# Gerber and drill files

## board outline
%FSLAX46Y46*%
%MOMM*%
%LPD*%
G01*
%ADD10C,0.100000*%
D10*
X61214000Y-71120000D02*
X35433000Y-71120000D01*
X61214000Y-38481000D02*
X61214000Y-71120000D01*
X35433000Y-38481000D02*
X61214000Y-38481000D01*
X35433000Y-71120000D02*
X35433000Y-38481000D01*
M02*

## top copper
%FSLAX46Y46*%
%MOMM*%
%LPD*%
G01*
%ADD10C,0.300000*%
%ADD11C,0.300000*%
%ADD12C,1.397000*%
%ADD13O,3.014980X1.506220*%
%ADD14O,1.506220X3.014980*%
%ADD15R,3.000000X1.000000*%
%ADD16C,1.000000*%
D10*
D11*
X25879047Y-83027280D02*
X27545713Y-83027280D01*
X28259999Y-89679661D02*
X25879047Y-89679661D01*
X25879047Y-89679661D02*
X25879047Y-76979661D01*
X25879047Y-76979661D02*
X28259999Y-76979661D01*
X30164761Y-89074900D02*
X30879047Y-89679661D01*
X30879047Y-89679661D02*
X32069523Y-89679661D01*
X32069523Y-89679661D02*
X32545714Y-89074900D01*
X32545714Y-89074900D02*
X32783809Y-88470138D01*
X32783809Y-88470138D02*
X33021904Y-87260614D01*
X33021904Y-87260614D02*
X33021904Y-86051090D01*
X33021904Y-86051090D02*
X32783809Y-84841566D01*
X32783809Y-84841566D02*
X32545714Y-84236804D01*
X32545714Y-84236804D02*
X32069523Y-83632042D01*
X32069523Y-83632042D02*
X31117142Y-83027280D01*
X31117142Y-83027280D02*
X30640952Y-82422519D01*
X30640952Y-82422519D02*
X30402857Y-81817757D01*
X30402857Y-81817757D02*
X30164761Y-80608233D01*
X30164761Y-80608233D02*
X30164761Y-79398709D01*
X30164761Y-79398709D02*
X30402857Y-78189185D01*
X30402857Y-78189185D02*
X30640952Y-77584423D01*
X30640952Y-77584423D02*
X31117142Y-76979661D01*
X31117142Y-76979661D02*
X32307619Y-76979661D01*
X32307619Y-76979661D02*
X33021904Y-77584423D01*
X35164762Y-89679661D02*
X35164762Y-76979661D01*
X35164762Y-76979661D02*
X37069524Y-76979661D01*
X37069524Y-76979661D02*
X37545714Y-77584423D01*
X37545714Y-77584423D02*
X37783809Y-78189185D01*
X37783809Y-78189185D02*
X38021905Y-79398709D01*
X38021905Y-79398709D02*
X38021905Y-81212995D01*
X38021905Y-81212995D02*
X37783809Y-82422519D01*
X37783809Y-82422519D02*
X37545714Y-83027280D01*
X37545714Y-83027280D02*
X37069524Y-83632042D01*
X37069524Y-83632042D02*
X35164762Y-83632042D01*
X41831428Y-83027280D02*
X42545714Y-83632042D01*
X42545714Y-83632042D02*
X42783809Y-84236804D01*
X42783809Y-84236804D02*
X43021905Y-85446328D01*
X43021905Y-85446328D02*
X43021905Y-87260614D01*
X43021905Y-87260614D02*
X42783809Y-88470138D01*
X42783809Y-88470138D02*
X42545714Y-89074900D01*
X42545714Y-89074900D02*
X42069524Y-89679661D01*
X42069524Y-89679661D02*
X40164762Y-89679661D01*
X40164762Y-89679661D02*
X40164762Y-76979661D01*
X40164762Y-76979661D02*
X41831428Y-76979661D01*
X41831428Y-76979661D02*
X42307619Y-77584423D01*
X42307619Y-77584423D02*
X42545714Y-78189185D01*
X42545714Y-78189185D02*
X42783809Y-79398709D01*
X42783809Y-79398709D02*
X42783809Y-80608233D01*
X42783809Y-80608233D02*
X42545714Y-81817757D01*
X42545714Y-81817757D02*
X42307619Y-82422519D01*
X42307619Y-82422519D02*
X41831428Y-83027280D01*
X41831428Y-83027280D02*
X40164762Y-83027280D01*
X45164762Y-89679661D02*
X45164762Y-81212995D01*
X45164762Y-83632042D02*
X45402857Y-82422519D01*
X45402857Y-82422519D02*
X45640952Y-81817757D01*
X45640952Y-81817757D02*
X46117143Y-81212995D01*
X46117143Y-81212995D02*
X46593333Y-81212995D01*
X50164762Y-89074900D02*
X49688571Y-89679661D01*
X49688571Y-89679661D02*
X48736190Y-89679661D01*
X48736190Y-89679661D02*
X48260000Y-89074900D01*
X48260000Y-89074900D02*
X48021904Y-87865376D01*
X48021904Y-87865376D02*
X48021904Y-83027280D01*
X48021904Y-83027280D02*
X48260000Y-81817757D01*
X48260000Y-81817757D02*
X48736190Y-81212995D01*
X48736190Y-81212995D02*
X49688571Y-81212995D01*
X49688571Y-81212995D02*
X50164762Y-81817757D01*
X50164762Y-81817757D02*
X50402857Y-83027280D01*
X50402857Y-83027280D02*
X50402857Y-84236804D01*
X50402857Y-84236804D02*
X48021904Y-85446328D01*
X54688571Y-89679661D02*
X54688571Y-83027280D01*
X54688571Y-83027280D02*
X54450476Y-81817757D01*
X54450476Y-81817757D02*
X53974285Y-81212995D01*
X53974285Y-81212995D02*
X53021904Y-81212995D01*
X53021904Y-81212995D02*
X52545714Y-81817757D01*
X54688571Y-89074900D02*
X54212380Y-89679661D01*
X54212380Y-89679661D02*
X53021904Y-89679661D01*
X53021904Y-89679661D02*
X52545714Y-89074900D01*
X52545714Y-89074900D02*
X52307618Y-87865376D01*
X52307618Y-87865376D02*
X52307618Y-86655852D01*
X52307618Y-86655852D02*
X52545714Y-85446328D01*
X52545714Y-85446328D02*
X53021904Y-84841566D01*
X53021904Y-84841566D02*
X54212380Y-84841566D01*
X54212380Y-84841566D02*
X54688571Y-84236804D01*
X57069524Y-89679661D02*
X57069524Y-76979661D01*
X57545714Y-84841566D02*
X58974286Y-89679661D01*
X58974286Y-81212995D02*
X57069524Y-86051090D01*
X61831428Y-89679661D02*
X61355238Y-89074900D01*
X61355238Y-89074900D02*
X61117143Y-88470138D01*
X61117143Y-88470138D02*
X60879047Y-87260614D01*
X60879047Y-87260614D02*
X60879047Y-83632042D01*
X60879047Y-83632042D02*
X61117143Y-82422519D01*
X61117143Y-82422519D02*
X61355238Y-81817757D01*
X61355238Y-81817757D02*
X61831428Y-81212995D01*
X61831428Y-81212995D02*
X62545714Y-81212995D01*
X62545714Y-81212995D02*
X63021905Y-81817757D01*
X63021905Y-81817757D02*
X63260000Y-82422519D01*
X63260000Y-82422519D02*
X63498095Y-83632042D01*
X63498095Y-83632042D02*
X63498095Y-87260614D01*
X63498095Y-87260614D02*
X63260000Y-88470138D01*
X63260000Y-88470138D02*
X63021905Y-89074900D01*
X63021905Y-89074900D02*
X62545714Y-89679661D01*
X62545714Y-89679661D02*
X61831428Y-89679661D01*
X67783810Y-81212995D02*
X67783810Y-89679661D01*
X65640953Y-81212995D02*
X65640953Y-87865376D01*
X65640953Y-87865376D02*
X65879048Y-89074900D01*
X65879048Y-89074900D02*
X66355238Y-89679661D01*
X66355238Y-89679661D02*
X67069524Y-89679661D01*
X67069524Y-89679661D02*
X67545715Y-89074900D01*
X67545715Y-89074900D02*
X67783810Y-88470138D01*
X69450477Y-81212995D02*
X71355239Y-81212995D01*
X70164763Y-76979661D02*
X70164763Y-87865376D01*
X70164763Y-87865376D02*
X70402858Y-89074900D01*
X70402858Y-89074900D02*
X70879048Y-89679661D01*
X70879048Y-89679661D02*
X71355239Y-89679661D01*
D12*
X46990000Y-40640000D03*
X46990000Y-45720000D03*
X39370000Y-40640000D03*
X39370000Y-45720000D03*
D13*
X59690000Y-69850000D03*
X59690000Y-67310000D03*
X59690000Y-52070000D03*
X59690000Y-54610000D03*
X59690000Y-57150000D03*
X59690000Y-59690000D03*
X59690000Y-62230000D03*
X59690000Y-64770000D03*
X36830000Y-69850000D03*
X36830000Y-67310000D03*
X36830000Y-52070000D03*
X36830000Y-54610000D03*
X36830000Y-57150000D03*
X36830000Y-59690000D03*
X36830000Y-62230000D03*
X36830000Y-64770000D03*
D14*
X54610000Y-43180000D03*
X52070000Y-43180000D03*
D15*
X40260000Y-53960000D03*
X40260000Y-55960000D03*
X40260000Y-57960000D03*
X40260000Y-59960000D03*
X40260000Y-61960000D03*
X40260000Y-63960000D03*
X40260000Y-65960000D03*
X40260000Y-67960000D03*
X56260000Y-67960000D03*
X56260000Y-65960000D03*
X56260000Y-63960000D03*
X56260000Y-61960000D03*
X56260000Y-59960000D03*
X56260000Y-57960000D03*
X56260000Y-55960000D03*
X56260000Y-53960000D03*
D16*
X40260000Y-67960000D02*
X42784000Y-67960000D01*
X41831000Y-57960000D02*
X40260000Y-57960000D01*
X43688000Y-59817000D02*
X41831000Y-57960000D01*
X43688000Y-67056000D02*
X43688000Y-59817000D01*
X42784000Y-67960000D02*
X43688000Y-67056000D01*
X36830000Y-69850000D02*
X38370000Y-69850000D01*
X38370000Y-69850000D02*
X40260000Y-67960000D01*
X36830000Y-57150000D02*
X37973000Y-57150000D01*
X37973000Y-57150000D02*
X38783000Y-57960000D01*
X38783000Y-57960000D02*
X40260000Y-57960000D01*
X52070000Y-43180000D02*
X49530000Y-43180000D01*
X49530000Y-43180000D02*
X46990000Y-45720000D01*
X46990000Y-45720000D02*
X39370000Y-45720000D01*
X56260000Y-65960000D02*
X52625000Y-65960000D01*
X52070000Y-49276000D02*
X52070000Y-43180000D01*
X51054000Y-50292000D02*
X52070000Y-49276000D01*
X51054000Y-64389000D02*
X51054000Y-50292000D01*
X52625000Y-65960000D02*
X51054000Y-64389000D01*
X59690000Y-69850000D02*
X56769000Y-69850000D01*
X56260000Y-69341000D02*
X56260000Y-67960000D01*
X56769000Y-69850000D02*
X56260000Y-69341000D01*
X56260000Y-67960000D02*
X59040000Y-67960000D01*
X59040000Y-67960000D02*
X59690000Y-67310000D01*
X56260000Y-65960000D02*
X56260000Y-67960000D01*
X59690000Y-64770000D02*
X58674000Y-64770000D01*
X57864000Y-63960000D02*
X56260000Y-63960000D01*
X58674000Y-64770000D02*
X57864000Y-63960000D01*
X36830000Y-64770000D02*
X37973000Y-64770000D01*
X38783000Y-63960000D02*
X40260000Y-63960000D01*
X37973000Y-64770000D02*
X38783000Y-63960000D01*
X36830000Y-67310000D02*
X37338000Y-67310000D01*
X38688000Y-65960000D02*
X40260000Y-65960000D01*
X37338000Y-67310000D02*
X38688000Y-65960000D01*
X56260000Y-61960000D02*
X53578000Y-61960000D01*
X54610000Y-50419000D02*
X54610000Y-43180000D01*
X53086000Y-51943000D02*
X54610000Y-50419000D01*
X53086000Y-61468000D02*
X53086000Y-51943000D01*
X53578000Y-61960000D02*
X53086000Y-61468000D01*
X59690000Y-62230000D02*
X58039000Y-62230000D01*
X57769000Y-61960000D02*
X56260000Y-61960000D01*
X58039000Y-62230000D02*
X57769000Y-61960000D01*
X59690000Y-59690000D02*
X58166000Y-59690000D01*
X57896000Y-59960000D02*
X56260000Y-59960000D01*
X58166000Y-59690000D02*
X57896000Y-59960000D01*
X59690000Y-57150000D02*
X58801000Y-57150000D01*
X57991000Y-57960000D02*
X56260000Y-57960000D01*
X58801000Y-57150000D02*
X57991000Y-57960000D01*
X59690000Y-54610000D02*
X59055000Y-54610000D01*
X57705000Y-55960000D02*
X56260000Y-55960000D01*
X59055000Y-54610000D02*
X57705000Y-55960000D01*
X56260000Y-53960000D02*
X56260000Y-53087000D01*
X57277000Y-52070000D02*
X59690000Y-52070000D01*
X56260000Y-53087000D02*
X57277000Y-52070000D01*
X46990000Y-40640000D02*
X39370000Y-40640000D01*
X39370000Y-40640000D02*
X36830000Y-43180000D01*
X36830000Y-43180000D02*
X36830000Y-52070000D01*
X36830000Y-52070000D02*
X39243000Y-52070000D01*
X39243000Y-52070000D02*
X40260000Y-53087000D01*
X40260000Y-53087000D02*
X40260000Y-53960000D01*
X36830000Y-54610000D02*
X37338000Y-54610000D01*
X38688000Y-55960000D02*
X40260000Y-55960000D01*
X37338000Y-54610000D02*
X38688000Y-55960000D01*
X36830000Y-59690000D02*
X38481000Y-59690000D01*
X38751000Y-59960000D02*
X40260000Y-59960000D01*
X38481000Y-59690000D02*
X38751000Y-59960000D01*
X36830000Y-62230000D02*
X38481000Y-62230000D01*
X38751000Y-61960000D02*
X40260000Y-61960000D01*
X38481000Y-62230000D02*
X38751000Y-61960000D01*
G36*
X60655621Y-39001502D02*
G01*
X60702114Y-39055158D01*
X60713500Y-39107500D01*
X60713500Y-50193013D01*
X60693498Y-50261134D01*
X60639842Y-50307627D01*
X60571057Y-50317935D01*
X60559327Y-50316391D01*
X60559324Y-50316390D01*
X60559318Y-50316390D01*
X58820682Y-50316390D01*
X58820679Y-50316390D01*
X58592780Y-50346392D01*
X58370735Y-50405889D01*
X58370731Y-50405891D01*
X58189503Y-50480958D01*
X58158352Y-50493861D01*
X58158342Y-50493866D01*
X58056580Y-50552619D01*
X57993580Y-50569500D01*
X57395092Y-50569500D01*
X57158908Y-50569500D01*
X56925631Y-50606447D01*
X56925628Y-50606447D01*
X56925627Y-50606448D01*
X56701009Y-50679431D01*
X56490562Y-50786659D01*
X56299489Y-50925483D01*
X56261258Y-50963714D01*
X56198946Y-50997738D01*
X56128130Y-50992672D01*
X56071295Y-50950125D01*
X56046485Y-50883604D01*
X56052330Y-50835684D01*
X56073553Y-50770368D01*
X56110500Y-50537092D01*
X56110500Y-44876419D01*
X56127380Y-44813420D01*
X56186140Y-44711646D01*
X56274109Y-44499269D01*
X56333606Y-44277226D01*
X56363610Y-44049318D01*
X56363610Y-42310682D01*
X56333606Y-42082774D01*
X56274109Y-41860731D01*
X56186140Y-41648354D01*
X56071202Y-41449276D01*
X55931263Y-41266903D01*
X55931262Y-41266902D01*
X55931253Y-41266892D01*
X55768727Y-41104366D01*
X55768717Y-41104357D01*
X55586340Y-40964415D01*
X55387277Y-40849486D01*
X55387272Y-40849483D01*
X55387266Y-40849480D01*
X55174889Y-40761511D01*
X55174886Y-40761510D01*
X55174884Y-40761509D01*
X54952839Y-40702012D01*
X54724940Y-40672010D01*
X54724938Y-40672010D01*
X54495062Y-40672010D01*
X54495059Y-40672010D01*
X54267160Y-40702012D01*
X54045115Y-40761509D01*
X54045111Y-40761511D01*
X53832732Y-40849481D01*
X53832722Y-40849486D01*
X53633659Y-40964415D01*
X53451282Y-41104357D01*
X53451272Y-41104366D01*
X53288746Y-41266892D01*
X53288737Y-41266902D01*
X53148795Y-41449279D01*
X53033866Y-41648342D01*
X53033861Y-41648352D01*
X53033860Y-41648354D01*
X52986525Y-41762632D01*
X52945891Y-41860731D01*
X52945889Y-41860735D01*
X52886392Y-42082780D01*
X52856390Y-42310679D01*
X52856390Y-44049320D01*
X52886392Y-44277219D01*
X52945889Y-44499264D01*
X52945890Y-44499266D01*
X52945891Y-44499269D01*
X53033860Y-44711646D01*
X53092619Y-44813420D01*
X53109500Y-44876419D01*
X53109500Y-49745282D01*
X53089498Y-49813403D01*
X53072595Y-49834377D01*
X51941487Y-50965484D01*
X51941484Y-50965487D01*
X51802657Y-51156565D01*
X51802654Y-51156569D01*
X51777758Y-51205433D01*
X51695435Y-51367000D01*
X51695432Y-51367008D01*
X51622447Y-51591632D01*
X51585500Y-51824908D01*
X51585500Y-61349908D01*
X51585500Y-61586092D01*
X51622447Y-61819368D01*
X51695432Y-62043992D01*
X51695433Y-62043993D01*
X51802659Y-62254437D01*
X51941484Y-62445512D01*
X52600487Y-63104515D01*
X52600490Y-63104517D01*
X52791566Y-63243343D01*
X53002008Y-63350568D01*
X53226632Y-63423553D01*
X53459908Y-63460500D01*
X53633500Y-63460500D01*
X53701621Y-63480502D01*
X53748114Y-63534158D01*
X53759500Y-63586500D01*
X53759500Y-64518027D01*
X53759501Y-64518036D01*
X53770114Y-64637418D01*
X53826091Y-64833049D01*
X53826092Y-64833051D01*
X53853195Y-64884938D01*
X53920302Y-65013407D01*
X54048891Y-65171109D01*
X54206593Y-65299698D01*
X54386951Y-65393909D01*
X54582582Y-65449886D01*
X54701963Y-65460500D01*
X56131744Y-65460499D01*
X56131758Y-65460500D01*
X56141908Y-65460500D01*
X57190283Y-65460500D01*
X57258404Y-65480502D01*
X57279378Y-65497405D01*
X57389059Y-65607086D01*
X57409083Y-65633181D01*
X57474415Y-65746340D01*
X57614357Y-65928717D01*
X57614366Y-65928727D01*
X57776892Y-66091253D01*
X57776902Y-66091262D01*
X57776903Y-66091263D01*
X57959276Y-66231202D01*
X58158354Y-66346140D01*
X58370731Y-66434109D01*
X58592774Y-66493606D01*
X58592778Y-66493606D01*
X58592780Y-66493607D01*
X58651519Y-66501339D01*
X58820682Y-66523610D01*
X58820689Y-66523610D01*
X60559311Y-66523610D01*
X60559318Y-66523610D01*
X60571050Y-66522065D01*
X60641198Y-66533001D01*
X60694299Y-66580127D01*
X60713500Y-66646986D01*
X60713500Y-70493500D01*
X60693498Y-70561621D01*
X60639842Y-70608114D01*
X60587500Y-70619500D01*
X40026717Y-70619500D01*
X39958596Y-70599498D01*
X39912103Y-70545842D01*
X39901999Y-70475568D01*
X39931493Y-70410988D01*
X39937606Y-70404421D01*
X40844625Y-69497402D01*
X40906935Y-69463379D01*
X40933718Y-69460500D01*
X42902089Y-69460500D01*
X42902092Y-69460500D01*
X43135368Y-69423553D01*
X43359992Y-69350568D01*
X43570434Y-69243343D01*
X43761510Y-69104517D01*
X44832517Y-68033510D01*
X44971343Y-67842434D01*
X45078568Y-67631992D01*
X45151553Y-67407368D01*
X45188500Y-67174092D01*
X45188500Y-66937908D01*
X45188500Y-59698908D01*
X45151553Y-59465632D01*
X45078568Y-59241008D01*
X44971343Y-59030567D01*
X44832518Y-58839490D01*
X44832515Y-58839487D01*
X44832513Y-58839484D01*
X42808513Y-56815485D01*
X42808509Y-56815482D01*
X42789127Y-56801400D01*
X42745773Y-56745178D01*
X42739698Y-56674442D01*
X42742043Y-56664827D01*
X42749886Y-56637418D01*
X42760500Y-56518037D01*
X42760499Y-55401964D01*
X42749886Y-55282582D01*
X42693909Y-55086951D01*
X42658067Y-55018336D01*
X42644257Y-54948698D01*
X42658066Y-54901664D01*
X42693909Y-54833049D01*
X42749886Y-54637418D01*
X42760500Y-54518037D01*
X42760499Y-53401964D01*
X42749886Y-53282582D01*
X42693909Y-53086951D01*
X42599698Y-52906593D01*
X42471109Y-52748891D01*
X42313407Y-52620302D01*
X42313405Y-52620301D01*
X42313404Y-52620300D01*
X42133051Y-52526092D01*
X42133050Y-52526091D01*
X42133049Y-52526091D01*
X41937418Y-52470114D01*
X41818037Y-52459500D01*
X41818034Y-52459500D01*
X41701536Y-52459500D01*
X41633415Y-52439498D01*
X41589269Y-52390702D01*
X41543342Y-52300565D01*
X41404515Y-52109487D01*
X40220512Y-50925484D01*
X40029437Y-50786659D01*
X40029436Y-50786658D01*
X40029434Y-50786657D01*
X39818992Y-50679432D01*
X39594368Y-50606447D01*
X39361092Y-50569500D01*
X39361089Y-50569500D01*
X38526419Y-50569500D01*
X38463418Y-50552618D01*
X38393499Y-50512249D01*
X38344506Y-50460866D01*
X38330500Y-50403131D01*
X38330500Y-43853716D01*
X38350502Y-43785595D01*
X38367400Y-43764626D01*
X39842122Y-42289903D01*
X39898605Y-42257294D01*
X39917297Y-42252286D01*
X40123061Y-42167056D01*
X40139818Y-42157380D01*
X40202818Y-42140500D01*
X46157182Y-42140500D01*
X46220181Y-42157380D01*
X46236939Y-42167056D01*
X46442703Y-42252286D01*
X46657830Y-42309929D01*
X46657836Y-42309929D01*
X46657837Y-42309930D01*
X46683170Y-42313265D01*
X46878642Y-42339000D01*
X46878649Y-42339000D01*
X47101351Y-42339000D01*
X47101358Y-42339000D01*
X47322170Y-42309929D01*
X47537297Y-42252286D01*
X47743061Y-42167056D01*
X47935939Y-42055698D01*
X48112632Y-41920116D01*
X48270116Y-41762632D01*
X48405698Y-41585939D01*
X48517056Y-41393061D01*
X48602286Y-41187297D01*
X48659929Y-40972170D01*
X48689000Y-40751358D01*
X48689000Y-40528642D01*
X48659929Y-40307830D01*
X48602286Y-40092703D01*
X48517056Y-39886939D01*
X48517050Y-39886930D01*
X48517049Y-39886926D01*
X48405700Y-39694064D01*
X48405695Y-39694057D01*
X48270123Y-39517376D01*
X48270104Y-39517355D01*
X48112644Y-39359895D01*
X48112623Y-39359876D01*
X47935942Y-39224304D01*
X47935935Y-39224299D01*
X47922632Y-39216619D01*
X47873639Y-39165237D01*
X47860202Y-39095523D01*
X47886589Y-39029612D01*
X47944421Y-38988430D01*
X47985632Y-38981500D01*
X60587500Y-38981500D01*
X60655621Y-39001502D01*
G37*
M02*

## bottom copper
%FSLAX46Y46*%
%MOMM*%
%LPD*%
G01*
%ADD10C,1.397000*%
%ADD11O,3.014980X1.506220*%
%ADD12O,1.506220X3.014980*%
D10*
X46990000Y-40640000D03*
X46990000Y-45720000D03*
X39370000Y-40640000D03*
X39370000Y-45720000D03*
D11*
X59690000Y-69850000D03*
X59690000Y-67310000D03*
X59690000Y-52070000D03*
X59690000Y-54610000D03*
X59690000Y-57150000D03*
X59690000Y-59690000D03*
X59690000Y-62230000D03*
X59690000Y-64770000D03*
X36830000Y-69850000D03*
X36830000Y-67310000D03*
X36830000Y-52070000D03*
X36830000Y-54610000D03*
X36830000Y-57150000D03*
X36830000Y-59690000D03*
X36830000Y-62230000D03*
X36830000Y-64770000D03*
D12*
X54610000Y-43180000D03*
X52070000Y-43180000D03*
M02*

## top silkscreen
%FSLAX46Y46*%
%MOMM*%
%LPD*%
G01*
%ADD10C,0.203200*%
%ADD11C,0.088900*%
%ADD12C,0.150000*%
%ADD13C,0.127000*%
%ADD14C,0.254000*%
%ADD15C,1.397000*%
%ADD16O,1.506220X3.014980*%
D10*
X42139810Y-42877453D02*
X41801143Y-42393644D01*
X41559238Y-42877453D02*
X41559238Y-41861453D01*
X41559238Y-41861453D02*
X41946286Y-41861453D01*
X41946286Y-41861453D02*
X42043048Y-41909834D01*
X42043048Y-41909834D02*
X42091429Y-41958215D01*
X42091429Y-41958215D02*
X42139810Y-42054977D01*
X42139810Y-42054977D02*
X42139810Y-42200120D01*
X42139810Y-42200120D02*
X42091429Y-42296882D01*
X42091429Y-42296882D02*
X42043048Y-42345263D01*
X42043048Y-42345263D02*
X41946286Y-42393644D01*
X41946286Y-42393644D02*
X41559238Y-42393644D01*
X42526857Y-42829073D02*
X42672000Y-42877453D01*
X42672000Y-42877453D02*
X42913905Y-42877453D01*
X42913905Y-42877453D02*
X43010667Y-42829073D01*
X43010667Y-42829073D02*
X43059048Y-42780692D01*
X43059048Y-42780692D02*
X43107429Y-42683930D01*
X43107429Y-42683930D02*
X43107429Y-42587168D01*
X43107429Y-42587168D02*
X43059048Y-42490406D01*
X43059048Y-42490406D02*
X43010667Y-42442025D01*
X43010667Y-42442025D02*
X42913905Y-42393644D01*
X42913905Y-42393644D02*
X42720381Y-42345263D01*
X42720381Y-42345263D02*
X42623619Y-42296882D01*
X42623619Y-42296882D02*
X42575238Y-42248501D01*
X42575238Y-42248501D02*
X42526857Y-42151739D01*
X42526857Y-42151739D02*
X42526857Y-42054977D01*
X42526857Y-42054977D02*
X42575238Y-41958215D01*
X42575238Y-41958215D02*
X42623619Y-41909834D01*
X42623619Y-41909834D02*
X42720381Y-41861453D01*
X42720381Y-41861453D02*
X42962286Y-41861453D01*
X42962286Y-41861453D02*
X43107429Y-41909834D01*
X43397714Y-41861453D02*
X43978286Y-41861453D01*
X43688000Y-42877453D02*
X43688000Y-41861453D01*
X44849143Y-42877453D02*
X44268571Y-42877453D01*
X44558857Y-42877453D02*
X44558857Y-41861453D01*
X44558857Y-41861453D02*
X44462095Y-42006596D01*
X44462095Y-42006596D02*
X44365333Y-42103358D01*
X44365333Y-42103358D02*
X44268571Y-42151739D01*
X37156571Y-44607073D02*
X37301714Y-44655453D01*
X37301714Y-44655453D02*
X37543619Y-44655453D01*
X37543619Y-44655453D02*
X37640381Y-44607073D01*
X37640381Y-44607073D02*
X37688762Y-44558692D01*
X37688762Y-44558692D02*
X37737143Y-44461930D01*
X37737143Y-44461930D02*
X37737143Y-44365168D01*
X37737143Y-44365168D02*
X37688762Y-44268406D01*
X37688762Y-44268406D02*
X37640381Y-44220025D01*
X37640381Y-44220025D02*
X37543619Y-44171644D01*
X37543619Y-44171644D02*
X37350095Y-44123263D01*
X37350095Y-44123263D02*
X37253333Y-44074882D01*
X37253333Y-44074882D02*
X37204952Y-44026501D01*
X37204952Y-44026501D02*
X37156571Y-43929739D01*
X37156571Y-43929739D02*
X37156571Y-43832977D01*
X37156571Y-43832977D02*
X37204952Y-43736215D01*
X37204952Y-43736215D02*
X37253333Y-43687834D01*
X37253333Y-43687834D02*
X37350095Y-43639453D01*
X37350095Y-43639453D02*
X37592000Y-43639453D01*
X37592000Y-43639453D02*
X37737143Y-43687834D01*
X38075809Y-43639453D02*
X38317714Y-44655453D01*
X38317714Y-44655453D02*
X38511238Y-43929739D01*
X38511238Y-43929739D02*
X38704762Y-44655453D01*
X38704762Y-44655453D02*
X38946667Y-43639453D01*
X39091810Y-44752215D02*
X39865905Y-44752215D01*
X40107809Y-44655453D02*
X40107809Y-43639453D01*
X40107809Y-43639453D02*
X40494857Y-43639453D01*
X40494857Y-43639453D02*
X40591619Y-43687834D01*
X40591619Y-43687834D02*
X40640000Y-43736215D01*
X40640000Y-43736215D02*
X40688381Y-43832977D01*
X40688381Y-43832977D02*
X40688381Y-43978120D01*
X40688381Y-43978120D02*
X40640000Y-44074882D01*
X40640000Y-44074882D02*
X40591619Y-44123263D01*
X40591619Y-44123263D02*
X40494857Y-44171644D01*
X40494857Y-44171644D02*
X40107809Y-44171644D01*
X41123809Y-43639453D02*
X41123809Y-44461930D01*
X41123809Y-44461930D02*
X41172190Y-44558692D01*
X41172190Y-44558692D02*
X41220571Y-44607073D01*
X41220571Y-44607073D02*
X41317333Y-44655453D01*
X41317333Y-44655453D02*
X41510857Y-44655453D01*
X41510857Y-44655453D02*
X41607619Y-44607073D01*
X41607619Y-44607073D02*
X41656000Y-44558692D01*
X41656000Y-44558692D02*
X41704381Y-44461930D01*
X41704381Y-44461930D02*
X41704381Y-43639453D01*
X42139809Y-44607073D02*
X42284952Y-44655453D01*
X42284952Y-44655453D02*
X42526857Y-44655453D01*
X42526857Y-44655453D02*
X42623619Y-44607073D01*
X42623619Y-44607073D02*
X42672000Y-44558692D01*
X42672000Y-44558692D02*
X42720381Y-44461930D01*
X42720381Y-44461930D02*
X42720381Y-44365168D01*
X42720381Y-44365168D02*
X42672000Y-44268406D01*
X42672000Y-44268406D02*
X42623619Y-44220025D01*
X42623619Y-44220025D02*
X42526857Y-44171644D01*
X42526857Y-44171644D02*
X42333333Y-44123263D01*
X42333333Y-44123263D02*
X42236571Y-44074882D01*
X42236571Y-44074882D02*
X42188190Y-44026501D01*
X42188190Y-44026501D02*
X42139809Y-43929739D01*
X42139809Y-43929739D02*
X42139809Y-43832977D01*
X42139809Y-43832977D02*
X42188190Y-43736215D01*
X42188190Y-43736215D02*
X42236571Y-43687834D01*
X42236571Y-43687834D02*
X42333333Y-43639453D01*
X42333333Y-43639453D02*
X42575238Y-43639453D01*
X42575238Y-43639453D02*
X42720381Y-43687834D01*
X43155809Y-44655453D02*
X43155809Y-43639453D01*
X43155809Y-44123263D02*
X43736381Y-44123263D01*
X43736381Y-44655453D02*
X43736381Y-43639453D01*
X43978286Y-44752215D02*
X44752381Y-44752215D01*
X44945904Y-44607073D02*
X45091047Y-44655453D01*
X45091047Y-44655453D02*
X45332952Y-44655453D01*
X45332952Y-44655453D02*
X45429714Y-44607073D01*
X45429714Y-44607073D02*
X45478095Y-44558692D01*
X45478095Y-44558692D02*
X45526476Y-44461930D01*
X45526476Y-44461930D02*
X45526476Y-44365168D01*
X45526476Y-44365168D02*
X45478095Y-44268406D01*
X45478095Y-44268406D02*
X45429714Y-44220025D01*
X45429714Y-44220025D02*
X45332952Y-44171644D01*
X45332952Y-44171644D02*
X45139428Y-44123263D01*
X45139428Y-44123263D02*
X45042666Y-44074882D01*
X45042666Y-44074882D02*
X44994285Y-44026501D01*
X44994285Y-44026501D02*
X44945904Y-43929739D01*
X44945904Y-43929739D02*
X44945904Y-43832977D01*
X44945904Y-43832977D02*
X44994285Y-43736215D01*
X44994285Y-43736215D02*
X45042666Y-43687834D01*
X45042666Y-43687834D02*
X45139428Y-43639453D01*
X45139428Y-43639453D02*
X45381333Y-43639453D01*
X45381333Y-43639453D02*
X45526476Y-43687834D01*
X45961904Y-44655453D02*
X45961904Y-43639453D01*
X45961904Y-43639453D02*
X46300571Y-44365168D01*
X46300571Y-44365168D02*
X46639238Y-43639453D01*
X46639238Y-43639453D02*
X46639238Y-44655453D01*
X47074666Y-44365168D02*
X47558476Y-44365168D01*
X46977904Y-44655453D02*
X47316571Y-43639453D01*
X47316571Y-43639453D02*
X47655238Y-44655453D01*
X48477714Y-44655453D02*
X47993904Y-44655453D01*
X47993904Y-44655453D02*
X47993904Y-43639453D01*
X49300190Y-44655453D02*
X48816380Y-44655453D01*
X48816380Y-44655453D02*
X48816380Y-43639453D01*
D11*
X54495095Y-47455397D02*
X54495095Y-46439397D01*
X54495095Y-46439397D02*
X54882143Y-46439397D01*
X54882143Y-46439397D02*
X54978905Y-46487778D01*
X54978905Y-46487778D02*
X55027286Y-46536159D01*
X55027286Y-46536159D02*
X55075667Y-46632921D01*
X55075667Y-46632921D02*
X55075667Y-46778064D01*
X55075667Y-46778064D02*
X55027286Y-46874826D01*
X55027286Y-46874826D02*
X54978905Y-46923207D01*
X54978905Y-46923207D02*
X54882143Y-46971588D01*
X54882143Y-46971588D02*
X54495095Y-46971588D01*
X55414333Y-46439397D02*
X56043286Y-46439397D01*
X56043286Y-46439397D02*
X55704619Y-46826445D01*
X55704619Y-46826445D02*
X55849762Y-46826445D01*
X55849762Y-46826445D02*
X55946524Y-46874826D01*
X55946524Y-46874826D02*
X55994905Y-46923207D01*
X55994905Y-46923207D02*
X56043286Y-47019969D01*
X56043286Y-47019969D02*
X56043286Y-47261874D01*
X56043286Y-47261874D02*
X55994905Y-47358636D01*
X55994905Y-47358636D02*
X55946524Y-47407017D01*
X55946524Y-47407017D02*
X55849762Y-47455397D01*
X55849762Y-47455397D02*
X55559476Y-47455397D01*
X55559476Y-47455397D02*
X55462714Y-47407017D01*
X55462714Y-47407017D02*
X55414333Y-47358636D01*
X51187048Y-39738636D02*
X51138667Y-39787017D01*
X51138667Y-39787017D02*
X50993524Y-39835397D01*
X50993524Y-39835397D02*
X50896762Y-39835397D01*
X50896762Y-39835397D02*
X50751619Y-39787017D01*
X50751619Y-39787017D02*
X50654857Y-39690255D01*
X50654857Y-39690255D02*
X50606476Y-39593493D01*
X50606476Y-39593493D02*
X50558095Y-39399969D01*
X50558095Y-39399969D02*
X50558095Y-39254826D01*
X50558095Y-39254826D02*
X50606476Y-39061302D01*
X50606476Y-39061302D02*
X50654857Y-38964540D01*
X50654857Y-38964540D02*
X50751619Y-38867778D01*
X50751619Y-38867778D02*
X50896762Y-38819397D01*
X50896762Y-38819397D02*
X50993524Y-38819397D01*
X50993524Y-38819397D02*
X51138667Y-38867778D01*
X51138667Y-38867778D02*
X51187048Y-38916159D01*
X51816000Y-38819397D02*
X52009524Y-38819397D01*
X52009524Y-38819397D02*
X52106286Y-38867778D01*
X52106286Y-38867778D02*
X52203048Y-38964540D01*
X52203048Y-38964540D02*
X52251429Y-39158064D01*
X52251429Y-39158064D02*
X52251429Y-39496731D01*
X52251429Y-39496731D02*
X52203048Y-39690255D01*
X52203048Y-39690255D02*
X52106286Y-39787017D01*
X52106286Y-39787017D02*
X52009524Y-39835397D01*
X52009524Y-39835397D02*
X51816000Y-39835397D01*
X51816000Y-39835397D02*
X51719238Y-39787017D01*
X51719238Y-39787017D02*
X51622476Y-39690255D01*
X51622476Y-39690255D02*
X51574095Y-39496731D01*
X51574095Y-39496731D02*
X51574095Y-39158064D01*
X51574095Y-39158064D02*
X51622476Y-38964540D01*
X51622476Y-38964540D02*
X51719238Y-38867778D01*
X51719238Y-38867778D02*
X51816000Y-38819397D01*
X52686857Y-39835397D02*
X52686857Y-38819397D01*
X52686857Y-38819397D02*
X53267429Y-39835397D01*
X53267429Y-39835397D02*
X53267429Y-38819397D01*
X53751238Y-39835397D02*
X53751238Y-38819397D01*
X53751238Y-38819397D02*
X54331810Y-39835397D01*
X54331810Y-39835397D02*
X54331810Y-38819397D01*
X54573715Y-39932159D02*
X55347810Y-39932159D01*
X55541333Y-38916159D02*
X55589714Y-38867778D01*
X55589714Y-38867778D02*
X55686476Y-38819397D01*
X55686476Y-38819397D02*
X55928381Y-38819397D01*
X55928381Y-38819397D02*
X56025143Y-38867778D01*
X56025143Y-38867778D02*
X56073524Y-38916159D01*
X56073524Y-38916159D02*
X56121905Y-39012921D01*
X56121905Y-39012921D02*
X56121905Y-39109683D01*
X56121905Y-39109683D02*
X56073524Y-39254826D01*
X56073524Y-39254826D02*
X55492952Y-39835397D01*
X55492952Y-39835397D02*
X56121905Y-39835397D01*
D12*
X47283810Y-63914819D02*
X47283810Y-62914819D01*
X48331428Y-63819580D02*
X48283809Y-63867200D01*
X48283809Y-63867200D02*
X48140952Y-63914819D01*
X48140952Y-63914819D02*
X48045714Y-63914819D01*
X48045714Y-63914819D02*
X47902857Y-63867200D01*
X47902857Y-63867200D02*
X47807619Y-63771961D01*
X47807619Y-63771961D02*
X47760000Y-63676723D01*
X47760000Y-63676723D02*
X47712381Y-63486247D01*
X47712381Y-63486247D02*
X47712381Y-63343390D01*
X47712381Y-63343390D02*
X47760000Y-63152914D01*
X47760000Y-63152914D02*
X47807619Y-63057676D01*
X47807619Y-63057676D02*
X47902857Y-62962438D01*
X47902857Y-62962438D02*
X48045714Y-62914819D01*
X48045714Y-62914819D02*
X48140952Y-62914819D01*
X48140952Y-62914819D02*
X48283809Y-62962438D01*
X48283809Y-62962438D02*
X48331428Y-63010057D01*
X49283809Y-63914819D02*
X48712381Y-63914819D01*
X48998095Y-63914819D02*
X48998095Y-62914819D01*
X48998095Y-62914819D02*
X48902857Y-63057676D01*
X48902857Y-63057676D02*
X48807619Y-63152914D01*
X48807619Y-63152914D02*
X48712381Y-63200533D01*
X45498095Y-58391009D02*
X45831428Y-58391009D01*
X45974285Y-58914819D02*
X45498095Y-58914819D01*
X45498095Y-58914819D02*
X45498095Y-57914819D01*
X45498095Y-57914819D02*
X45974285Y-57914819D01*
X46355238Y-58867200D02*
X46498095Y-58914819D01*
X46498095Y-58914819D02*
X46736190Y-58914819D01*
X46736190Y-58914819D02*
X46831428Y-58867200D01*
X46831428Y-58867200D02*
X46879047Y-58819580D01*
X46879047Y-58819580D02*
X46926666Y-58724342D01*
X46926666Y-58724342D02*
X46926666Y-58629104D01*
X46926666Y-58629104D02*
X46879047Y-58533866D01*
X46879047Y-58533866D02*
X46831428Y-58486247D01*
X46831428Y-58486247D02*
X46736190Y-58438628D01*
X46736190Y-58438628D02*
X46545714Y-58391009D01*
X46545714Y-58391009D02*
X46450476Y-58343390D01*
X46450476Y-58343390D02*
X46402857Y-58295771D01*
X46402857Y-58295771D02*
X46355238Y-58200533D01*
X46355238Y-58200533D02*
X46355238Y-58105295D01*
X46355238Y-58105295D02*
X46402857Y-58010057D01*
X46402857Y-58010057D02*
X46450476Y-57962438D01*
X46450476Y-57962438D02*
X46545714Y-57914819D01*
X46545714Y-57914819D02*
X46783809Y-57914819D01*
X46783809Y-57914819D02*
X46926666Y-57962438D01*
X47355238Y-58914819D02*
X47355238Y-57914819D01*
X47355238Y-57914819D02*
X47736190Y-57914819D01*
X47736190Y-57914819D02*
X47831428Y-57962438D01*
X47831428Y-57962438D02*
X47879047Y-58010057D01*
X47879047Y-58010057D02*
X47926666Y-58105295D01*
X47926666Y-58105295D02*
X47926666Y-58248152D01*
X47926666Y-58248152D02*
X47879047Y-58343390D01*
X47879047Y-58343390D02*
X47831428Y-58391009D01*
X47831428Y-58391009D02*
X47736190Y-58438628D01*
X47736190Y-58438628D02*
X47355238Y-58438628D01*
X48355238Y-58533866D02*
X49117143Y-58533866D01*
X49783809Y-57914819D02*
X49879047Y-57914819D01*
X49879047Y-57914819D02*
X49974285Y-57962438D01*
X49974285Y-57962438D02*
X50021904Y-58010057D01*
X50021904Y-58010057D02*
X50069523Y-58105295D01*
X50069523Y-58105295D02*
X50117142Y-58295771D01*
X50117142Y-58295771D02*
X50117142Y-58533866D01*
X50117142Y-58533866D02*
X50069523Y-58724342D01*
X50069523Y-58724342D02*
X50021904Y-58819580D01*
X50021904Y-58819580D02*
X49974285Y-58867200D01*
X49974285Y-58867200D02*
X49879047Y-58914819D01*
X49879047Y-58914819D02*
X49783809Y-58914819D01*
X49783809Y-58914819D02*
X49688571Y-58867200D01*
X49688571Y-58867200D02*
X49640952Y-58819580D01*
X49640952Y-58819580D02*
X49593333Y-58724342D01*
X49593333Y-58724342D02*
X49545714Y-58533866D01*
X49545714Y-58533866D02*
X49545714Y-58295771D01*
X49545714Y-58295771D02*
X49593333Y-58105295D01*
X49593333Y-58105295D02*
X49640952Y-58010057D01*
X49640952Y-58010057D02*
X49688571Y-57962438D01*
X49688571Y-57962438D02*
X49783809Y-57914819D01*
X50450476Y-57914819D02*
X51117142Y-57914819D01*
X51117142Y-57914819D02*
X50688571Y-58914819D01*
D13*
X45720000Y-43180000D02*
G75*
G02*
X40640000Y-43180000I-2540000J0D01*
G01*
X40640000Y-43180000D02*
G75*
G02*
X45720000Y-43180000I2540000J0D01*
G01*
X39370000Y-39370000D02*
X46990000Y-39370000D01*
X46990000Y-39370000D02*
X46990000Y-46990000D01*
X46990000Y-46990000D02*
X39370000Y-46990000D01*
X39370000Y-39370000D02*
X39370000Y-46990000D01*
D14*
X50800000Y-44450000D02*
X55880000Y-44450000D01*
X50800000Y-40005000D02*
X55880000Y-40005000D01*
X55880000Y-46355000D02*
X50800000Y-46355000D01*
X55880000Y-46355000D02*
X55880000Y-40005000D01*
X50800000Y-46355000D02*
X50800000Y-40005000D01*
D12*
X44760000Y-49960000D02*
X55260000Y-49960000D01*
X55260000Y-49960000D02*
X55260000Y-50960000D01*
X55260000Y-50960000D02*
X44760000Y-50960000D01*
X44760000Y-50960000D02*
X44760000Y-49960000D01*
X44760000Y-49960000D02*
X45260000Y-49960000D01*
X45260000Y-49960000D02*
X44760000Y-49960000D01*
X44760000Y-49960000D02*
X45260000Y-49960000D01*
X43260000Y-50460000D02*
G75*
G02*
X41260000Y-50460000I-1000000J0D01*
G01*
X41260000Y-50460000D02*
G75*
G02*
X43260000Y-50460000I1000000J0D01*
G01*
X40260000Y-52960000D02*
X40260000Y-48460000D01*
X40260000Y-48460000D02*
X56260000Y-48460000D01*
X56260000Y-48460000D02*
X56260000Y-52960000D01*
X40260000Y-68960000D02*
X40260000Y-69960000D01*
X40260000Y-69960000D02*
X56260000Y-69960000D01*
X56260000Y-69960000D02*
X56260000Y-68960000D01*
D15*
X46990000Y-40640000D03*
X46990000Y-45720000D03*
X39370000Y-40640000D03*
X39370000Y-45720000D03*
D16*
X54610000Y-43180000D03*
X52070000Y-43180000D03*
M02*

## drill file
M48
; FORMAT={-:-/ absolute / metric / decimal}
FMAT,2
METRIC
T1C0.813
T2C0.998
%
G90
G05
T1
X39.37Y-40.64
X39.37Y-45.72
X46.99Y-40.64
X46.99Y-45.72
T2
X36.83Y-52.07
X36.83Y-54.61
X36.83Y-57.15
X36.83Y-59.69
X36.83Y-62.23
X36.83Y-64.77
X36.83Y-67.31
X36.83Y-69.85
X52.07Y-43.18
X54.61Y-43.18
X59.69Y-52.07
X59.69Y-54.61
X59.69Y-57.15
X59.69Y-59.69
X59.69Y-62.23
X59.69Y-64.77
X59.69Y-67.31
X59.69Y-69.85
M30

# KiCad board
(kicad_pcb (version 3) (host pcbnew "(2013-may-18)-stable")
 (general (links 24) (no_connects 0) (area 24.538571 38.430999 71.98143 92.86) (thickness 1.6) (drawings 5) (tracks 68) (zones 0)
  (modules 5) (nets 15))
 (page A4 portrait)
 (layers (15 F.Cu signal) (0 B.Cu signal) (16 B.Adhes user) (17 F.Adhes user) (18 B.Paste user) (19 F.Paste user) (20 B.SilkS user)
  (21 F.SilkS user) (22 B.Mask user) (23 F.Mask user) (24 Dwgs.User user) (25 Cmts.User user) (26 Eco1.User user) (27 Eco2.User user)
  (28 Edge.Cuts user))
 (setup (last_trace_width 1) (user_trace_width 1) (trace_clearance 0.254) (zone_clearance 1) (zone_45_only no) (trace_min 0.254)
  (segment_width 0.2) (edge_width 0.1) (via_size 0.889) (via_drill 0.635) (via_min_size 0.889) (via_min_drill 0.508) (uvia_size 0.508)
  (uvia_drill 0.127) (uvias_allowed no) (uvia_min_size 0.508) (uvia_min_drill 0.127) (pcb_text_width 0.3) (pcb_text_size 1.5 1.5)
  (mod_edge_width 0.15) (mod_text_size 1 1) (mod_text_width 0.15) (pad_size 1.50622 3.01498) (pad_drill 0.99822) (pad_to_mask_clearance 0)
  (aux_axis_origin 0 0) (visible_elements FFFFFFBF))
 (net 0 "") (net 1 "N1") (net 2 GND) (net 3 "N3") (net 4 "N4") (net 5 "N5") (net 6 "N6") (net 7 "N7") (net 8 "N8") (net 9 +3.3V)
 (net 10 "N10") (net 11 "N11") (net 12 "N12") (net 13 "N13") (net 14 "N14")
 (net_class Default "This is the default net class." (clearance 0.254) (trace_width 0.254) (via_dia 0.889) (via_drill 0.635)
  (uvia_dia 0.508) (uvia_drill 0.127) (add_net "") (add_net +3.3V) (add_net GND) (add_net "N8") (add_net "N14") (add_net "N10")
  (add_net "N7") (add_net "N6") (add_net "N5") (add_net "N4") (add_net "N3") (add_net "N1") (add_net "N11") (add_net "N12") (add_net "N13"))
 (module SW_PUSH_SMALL (layer F.Cu) (at 43.18 43.18)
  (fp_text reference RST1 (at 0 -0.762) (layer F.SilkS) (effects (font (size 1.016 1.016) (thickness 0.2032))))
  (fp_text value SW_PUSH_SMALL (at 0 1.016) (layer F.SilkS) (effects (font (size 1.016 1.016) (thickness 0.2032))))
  (fp_circle (center 0 0) (end 0 -2.54) (layer F.SilkS) (width 0.127))
  (fp_line (start -3.81 -3.81) (end 3.81 -3.81) (layer F.SilkS) (width 0.127))
  (fp_line (start 3.81 -3.81) (end 3.81 3.81) (layer F.SilkS) (width 0.127))
  (fp_line (start 3.81 3.81) (end -3.81 3.81) (layer F.SilkS) (width 0.127))
  (fp_line (start -3.81 -3.81) (end -3.81 3.81) (layer F.SilkS) (width 0.127))
  (pad 1 thru_hole circle (at 3.81 -2.54) (size 1.397 1.397) (drill 0.8128) (layers *.Cu *.Mask F.SilkS) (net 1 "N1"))
  (pad 2 thru_hole circle (at 3.81 2.54) (size 1.397 1.397) (drill 0.8128) (layers *.Cu *.Mask F.SilkS) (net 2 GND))
  (pad 1 thru_hole circle (at -3.81 -2.54) (size 1.397 1.397) (drill 0.8128) (layers *.Cu *.Mask F.SilkS) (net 1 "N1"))
  (pad 2 thru_hole circle (at -3.81 2.54) (size 1.397 1.397) (drill 0.8128) (layers *.Cu *.Mask F.SilkS) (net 2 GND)))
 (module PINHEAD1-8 (layer B.Cu) (at 59.69 58.42 270)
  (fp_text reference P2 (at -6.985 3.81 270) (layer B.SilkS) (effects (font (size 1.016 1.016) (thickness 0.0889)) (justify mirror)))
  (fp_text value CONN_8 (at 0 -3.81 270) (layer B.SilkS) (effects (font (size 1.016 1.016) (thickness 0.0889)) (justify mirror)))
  (pad 8 thru_hole oval (at 11.43 0 270) (size 1.50622 3.01498) (drill 0.99822) (layers *.Cu B.Paste B.SilkS B.Mask) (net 2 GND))
  (pad 7 thru_hole oval (at 8.89 0 270) (size 1.50622 3.01498) (drill 0.99822) (layers *.Cu B.Paste B.SilkS B.Mask) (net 2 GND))
  (pad 1 thru_hole oval (at -6.35 0 270) (size 1.50622 3.01498) (drill 0.99822) (layers *.Cu B.Paste B.SilkS B.Mask) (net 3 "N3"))
  (pad 2 thru_hole oval (at -3.81 0 270) (size 1.50622 3.01498) (drill 0.99822) (layers *.Cu B.Paste B.SilkS B.Mask) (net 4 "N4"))
  (pad 3 thru_hole oval (at -1.27 0 270) (size 1.50622 3.01498) (drill 0.99822) (layers *.Cu B.Paste B.SilkS B.Mask) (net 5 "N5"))
  (pad 4 thru_hole oval (at 1.27 0 270) (size 1.50622 3.01498) (drill 0.99822) (layers *.Cu B.Paste B.SilkS B.Mask) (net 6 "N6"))
  (pad 5 thru_hole oval (at 3.81 0 270) (size 1.50622 3.01498) (drill 0.99822) (layers *.Cu B.Paste B.SilkS B.Mask) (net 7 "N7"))
  (pad 6 thru_hole oval (at 6.35 0 270) (size 1.50622 3.01498) (drill 0.99822) (layers *.Cu B.Paste B.SilkS B.Mask) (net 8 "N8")))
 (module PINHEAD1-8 (layer B.Cu) (at 36.83 58.42 270)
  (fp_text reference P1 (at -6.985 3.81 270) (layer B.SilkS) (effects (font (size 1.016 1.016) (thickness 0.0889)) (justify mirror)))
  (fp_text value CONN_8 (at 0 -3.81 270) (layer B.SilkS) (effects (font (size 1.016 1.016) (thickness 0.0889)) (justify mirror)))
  (pad 8 thru_hole oval (at 11.43 0 270) (size 1.50622 3.01498) (drill 0.99822) (layers *.Cu B.Paste B.SilkS B.Mask) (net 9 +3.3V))
  (pad 7 thru_hole oval (at 8.89 0 270) (size 1.50622 3.01498) (drill 0.99822) (layers *.Cu B.Paste B.SilkS B.Mask) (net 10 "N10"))
  (pad 1 thru_hole oval (at -6.35 0 270) (size 1.50622 3.01498) (drill 0.99822) (layers *.Cu B.Paste B.SilkS B.Mask) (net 1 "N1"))
  (pad 2 thru_hole oval (at -3.81 0 270) (size 1.50622 3.01498) (drill 0.99822) (layers *.Cu B.Paste B.SilkS B.Mask) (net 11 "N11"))
  (pad 3 thru_hole oval (at -1.27 0 270) (size 1.50622 3.01498) (drill 0.99822) (layers *.Cu B.Paste B.SilkS B.Mask) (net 9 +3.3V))
  (pad 4 thru_hole oval (at 1.27 0 270) (size 1.50622 3.01498) (drill 0.99822) (layers *.Cu B.Paste B.SilkS B.Mask) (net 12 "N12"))
  (pad 5 thru_hole oval (at 3.81 0 270) (size 1.50622 3.01498) (drill 0.99822) (layers *.Cu B.Paste B.SilkS B.Mask) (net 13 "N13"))
  (pad 6 thru_hole oval (at 6.35 0 270) (size 1.50622 3.01498) (drill 0.99822) (layers *.Cu B.Paste B.SilkS B.Mask) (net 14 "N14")))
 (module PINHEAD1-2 (layer F.Cu) (at 53.34 43.18 180)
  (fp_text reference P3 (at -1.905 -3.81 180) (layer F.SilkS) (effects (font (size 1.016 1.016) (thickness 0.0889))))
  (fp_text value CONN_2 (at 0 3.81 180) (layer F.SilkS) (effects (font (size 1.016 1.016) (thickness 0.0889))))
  (fp_line (start 2.54 -1.27) (end -2.54 -1.27) (layer F.SilkS) (width 0.254))
  (fp_line (start 2.54 3.175) (end -2.54 3.175) (layer F.SilkS) (width 0.254))
  (fp_line (start -2.54 -3.175) (end 2.54 -3.175) (layer F.SilkS) (width 0.254))
  (fp_line (start -2.54 -3.175) (end -2.54 3.175) (layer F.SilkS) (width 0.254))
  (fp_line (start 2.54 -3.175) (end 2.54 3.175) (layer F.SilkS) (width 0.254))
  (pad 1 thru_hole oval (at -1.27 0 180) (size 1.50622 3.01498) (drill 0.99822) (layers *.Cu F.Paste F.SilkS F.Mask) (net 7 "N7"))
  (pad 2 thru_hole oval (at 1.27 0 180) (size 1.50622 3.01498) (drill 0.99822) (layers *.Cu F.Paste F.SilkS F.Mask) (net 2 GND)))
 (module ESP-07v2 (layer F.Cu) (at 48.26 60.96)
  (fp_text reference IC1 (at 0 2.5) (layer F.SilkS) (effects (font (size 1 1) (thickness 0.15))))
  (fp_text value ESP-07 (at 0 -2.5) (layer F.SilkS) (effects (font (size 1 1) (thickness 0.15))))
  (fp_line (start -3.5 -11) (end 7 -11) (layer F.SilkS) (width 0.15))
  (fp_line (start 7 -11) (end 7 -10) (layer F.SilkS) (width 0.15))
  (fp_line (start 7 -10) (end -3.5 -10) (layer F.SilkS) (width 0.15))
  (fp_line (start -3.5 -10) (end -3.5 -11) (layer F.SilkS) (width 0.15))
  (fp_line (start -3.5 -11) (end -3 -11) (layer F.SilkS) (width 0.15))
  (fp_line (start -3 -11) (end -3.5 -11) (layer F.SilkS) (width 0.15))
  (fp_line (start -3.5 -11) (end -3 -11) (layer F.SilkS) (width 0.15))
  (fp_circle (center -6 -10.5) (end -6 -9.5) (layer F.SilkS) (width 0.15))
  (fp_line (start -8 -8) (end -8 -12.5) (layer F.SilkS) (width 0.15))
  (fp_line (start -8 -12.5) (end 8 -12.5) (layer F.SilkS) (width 0.15))
  (fp_line (start 8 -12.5) (end 8 -8) (layer F.SilkS) (width 0.15))
  (fp_line (start -8 8) (end -8 9) (layer F.SilkS) (width 0.15))
  (fp_line (start -8 9) (end 8 9) (layer F.SilkS) (width 0.15)) (fp_line (start 8 9) (end 8 8) (layer F.SilkS) (width 0.15))
  (pad 1 smd rect (at -8 -7) (size 3 1) (layers F.Cu F.Paste F.Mask) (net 1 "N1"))
  (pad 2 smd rect (at -8 -5) (size 3 1) (layers F.Cu F.Paste F.Mask) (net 11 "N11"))
  (pad 3 smd rect (at -8 -3) (size 3 1) (layers F.Cu F.Paste F.Mask) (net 9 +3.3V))
  (pad 4 smd rect (at -8 -1) (size 3 1) (layers F.Cu F.Paste F.Mask) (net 12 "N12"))
  (pad 5 smd rect (at -8 1) (size 3 1) (layers F.Cu F.Paste F.Mask) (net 13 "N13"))
  (pad 6 smd rect (at -8 3) (size 3 1) (layers F.Cu F.Paste F.Mask) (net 14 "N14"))
  (pad 7 smd rect (at -8 5) (size 3 1) (layers F.Cu F.Paste F.Mask) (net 10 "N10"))
  (pad 8 smd rect (at -8 7) (size 3 1) (layers F.Cu F.Paste F.Mask) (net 9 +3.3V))
  (pad 9 smd rect (at 8 7) (size 3 1) (layers F.Cu F.Paste F.Mask) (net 2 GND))
  (pad 10 smd rect (at 8 5) (size 3 1) (layers F.Cu F.Paste F.Mask) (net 2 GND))
  (pad 11 smd rect (at 8 3) (size 3 1) (layers F.Cu F.Paste F.Mask) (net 8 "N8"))
  (pad 12 smd rect (at 8 1) (size 3 1) (layers F.Cu F.Paste F.Mask) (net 7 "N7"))
  (pad 13 smd rect (at 8 -1) (size 3 1) (layers F.Cu F.Paste F.Mask) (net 6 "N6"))
  (pad 14 smd rect (at 8 -3) (size 3 1) (layers F.Cu F.Paste F.Mask) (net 5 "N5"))
  (pad 15 smd rect (at 8 -5) (size 3 1) (layers F.Cu F.Paste F.Mask) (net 4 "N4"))
  (pad 16 smd rect (at 8 -7) (size 3 1) (layers F.Cu F.Paste F.Mask) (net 3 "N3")))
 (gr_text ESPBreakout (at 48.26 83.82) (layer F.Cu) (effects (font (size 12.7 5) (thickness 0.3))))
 (gr_line (start 61.214 71.12) (end 35.433 71.12) (angle 90) (layer Edge.Cuts) (width 0.1))
 (gr_line (start 61.214 38.481) (end 61.214 71.12) (angle 90) (layer Edge.Cuts) (width 0.1))
 (gr_line (start 35.433 38.481) (end 61.214 38.481) (angle 90) (layer Edge.Cuts) (width 0.1))
 (gr_line (start 35.433 71.12) (end 35.433 38.481) (angle 90) (layer Edge.Cuts) (width 0.1))
 (segment (start 40.26 67.96) (end 42.784 67.96) (width 1) (layer F.Cu) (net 9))
 (segment (start 41.831 57.96) (end 40.26 57.96) (width 1) (layer F.Cu) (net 9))
 (segment (start 43.688 59.817) (end 41.831 57.96) (width 1) (layer F.Cu) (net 9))
 (segment (start 43.688 67.056) (end 43.688 59.817) (width 1) (layer F.Cu) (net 9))
 (segment (start 42.784 67.96) (end 43.688 67.056) (width 1) (layer F.Cu) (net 9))
 (segment (start 36.83 69.85) (end 38.37 69.85) (width 1) (layer F.Cu) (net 9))
 (segment (start 38.37 69.85) (end 40.26 67.96) (width 1) (layer F.Cu) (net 9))
 (segment (start 36.83 57.15) (end 37.973 57.15) (width 1) (layer F.Cu) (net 9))
 (segment (start 37.973 57.15) (end 38.783 57.96) (width 1) (layer F.Cu) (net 9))
 (segment (start 38.783 57.96) (end 40.26 57.96) (width 1) (layer F.Cu) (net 9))
 (segment (start 52.07 43.18) (end 49.53 43.18) (width 1) (layer F.Cu) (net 2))
 (segment (start 49.53 43.18) (end 46.99 45.72) (width 1) (layer F.Cu) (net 2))
 (segment (start 46.99 45.72) (end 39.37 45.72) (width 1) (layer F.Cu) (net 2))
 (segment (start 56.26 65.96) (end 52.625 65.96) (width 1) (layer F.Cu) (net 2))
 (segment (start 52.07 49.276) (end 52.07 43.18) (width 1) (layer F.Cu) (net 2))
 (segment (start 51.054 50.292) (end 52.07 49.276) (width 1) (layer F.Cu) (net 2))
 (segment (start 51.054 64.389) (end 51.054 50.292) (width 1) (layer F.Cu) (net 2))
 (segment (start 52.625 65.96) (end 51.054 64.389) (width 1) (layer F.Cu) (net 2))
 (segment (start 59.69 69.85) (end 56.769 69.85) (width 1) (layer F.Cu) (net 2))
 (segment (start 56.26 69.341) (end 56.26 67.96) (width 1) (layer F.Cu) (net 2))
 (segment (start 56.769 69.85) (end 56.26 69.341) (width 1) (layer F.Cu) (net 2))
 (segment (start 56.26 67.96) (end 59.04 67.96) (width 1) (layer F.Cu) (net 2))
 (segment (start 59.04 67.96) (end 59.69 67.31) (width 1) (layer F.Cu) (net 2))
 (segment (start 56.26 65.96) (end 56.26 67.96) (width 1) (layer F.Cu) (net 2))
 (segment (start 59.69 64.77) (end 58.674 64.77) (width 1) (layer F.Cu) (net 8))
 (segment (start 57.864 63.96) (end 56.26 63.96) (width 1) (layer F.Cu) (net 8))
 (segment (start 58.674 64.77) (end 57.864 63.96) (width 1) (layer F.Cu) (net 8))
 (segment (start 36.83 64.77) (end 37.973 64.77) (width 1) (layer F.Cu) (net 14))
 (segment (start 38.783 63.96) (end 40.26 63.96) (width 1) (layer F.Cu) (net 14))
 (segment (start 37.973 64.77) (end 38.783 63.96) (width 1) (layer F.Cu) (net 14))
 (segment (start 36.83 67.31) (end 37.338 67.31) (width 1) (layer F.Cu) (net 10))
 (segment (start 38.688 65.96) (end 40.26 65.96) (width 1) (layer F.Cu) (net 10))
 (segment (start 37.338 67.31) (end 38.688 65.96) (width 1) (layer F.Cu) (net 10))
 (segment (start 56.26 61.96) (end 53.578 61.96) (width 1) (layer F.Cu) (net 7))
 (segment (start 54.61 50.419) (end 54.61 43.18) (width 1) (layer F.Cu) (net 7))
 (segment (start 53.086 51.943) (end 54.61 50.419) (width 1) (layer F.Cu) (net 7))
 (segment (start 53.086 61.468) (end 53.086 51.943) (width 1) (layer F.Cu) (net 7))
 (segment (start 53.578 61.96) (end 53.086 61.468) (width 1) (layer F.Cu) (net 7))
 (segment (start 59.69 62.23) (end 58.039 62.23) (width 1) (layer F.Cu) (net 7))
 (segment (start 57.769 61.96) (end 56.26 61.96) (width 1) (layer F.Cu) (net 7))
 (segment (start 58.039 62.23) (end 57.769 61.96) (width 1) (layer F.Cu) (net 7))
 (segment (start 59.69 59.69) (end 58.166 59.69) (width 1) (layer F.Cu) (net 6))
 (segment (start 57.896 59.96) (end 56.26 59.96) (width 1) (layer F.Cu) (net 6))
 (segment (start 58.166 59.69) (end 57.896 59.96) (width 1) (layer F.Cu) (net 6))
 (segment (start 59.69 57.15) (end 58.801 57.15) (width 1) (layer F.Cu) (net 5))
 (segment (start 57.991 57.96) (end 56.26 57.96) (width 1) (layer F.Cu) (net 5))
 (segment (start 58.801 57.15) (end 57.991 57.96) (width 1) (layer F.Cu) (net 5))
 (segment (start 59.69 54.61) (end 59.055 54.61) (width 1) (layer F.Cu) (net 4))
 (segment (start 57.705 55.96) (end 56.26 55.96) (width 1) (layer F.Cu) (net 4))
 (segment (start 59.055 54.61) (end 57.705 55.96) (width 1) (layer F.Cu) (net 4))
 (segment (start 56.26 53.96) (end 56.26 53.087) (width 1) (layer F.Cu) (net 3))
 (segment (start 57.277 52.07) (end 59.69 52.07) (width 1) (layer F.Cu) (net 3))
 (segment (start 56.26 53.087) (end 57.277 52.07) (width 1) (layer F.Cu) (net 3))
 (segment (start 46.99 40.64) (end 39.37 40.64) (width 1) (layer F.Cu) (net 1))
 (segment (start 39.37 40.64) (end 36.83 43.18) (width 1) (layer F.Cu) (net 1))
 (segment (start 36.83 43.18) (end 36.83 52.07) (width 1) (layer F.Cu) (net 1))
 (segment (start 36.83 52.07) (end 39.243 52.07) (width 1) (layer F.Cu) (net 1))
 (segment (start 39.243 52.07) (end 40.26 53.087) (width 1) (layer F.Cu) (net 1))
 (segment (start 40.26 53.087) (end 40.26 53.96) (width 1) (layer F.Cu) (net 1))
 (segment (start 36.83 54.61) (end 37.338 54.61) (width 1) (layer F.Cu) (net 11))
 (segment (start 38.688 55.96) (end 40.26 55.96) (width 1) (layer F.Cu) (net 11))
 (segment (start 37.338 54.61) (end 38.688 55.96) (width 1) (layer F.Cu) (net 11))
 (segment (start 36.83 59.69) (end 38.481 59.69) (width 1) (layer F.Cu) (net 12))
 (segment (start 38.751 59.96) (end 40.26 59.96) (width 1) (layer F.Cu) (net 12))
 (segment (start 38.481 59.69) (end 38.751 59.96) (width 1) (layer F.Cu) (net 12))
 (segment (start 36.83 62.23) (end 38.481 62.23) (width 1) (layer F.Cu) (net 13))
 (segment (start 38.751 61.96) (end 40.26 61.96) (width 1) (layer F.Cu) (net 13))
 (segment (start 38.481 62.23) (end 38.751 61.96) (width 1) (layer F.Cu) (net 13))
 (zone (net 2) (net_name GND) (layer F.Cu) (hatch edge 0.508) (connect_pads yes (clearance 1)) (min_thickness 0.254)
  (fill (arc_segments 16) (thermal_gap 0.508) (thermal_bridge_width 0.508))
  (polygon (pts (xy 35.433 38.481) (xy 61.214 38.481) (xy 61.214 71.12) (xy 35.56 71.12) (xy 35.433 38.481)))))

